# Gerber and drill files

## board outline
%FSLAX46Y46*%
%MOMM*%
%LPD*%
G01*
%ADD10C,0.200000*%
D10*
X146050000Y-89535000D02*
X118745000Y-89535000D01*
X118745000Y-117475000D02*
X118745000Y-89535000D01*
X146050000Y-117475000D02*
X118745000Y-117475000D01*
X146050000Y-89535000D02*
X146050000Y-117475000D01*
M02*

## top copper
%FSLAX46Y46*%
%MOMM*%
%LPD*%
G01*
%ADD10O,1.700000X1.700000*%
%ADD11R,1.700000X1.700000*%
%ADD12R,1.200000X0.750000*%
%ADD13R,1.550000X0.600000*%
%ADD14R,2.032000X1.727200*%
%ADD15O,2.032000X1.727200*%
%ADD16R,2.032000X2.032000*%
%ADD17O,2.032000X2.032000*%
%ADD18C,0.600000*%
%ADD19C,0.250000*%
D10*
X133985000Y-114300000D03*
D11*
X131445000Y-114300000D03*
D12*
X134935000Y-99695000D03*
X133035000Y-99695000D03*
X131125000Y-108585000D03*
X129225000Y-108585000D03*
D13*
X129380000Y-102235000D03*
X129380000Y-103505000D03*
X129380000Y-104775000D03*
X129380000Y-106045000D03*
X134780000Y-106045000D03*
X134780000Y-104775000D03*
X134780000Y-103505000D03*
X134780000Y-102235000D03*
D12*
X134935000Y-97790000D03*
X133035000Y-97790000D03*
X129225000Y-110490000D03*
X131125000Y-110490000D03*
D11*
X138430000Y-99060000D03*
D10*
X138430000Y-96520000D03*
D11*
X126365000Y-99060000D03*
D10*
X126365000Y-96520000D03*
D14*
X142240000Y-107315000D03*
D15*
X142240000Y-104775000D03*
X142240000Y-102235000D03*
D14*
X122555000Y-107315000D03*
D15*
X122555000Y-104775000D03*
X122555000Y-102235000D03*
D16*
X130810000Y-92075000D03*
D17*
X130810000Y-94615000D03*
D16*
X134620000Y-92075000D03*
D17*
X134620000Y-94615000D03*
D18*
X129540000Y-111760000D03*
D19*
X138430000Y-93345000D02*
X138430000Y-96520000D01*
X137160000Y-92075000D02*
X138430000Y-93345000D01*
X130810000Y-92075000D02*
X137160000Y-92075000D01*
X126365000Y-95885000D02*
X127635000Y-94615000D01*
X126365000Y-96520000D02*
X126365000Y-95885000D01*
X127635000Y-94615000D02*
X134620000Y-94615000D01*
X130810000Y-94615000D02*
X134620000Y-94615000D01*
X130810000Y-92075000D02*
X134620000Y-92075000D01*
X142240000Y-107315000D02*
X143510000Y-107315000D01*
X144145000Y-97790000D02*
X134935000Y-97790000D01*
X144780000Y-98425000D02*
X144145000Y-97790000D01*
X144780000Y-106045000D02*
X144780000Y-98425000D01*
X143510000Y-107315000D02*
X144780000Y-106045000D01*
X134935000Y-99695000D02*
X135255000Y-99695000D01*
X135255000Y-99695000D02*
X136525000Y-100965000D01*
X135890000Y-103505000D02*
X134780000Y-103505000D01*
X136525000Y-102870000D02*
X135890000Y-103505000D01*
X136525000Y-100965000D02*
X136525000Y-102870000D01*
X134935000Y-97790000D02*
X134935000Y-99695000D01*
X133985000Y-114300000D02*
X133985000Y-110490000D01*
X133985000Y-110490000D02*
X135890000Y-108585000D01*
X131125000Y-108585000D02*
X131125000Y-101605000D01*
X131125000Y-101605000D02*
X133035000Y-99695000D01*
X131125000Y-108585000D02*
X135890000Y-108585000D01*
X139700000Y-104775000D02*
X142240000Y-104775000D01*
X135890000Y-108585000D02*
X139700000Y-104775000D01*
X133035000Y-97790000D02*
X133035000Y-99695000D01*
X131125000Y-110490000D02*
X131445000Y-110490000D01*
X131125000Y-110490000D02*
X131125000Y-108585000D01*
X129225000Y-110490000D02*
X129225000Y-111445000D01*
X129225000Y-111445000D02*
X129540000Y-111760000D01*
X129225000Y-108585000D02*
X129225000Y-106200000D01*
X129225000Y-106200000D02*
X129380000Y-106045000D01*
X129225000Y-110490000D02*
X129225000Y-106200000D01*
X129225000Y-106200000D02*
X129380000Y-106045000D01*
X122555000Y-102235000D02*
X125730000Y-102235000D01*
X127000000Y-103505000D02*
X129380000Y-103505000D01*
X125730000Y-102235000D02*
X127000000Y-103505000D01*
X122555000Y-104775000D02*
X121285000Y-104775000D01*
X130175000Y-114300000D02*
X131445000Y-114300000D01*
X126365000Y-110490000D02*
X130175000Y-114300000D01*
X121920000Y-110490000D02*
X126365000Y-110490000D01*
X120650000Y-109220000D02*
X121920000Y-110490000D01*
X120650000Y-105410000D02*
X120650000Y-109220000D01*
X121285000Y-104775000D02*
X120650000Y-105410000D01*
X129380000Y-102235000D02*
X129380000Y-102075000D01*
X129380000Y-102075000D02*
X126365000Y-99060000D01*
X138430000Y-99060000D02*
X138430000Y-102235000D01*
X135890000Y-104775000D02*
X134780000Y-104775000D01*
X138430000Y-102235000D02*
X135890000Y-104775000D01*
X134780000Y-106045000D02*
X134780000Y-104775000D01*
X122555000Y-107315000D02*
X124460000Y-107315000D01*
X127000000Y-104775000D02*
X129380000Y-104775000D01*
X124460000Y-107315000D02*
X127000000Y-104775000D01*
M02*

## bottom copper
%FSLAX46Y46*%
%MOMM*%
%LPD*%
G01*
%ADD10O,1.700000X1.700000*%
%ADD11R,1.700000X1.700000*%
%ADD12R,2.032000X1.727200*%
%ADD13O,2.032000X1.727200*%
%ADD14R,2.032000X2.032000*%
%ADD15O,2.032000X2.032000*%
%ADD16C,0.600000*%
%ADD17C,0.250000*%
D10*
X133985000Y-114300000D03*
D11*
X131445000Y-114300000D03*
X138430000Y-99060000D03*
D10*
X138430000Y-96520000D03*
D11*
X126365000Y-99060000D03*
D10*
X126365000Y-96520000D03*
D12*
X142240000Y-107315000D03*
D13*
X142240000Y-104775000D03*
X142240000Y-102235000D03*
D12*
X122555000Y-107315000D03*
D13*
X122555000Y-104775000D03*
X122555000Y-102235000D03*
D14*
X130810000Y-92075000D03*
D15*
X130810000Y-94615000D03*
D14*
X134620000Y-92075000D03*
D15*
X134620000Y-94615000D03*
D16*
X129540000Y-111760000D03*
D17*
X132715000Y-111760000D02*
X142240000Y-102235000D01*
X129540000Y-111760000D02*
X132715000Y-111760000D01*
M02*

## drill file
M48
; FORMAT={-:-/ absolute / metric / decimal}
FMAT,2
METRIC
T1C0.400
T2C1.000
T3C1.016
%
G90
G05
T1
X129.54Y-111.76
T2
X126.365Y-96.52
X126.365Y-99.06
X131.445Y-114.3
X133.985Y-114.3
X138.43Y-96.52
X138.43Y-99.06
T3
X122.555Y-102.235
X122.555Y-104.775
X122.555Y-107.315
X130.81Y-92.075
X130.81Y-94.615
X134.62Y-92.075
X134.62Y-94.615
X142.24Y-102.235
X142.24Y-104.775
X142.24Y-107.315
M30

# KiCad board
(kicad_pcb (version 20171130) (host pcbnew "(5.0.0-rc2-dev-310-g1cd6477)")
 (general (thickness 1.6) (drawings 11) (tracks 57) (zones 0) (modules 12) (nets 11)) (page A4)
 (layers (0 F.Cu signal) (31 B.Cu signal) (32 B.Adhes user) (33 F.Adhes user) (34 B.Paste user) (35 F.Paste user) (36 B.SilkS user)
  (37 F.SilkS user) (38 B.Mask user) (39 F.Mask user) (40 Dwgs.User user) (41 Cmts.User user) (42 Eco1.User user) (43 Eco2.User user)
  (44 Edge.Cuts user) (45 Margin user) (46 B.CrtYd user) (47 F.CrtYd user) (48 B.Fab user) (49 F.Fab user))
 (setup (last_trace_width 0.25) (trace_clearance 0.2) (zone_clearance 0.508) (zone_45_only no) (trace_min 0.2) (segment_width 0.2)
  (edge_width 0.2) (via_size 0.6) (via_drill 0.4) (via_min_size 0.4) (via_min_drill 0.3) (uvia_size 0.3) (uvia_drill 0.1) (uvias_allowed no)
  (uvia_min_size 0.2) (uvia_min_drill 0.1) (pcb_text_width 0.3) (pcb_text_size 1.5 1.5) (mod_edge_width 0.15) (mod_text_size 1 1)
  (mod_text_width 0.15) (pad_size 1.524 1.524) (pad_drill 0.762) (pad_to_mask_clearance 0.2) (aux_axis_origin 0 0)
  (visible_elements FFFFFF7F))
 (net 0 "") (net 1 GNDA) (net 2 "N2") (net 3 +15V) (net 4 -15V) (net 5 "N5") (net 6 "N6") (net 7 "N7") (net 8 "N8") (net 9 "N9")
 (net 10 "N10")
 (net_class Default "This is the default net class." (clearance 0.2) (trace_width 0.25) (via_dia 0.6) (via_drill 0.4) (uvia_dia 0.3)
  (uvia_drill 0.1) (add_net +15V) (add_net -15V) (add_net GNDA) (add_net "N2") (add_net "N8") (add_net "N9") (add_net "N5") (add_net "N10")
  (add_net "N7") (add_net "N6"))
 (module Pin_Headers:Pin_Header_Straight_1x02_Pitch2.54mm (layer F.Cu) (at 131.445 114.3 90)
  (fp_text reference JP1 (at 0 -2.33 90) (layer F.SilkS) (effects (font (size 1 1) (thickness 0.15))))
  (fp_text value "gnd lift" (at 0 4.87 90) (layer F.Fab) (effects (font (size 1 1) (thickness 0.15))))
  (pad 2 thru_hole oval (at 0 2.54 90) (size 1.7 1.7) (drill 1) (layers *.Cu *.Mask) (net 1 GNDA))
  (pad 1 thru_hole rect (at 0 0 90) (size 1.7 1.7) (drill 1) (layers *.Cu *.Mask) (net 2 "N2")))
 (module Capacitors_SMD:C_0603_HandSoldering (layer F.Cu) (at 133.985 99.695 180)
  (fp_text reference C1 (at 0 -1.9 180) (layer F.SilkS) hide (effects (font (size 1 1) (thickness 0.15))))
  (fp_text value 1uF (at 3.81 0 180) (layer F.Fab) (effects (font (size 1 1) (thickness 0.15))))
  (pad 1 smd rect (at -0.95 0 180) (size 1.2 0.75) (layers F.Cu F.Paste F.Mask) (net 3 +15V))
  (pad 2 smd rect (at 0.95 0 180) (size 1.2 0.75) (layers F.Cu F.Paste F.Mask) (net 1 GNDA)))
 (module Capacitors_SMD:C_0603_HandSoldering (layer F.Cu) (at 130.175 108.585 180)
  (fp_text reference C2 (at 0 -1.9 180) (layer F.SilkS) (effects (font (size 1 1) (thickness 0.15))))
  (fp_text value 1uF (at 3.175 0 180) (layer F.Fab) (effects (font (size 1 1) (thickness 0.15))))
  (pad 1 smd rect (at -0.95 0 180) (size 1.2 0.75) (layers F.Cu F.Paste F.Mask) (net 1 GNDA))
  (pad 2 smd rect (at 0.95 0 180) (size 1.2 0.75) (layers F.Cu F.Paste F.Mask) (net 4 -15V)))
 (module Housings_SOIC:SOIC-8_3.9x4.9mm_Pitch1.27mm (layer F.Cu) (at 132.08 104.14)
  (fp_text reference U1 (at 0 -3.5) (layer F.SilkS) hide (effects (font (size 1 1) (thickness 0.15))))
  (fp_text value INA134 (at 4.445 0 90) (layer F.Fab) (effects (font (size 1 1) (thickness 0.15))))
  (pad 1 smd rect (at -2.7 -1.905) (size 1.55 0.6) (layers F.Cu F.Paste F.Mask) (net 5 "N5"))
  (pad 2 smd rect (at -2.7 -0.635) (size 1.55 0.6) (layers F.Cu F.Paste F.Mask) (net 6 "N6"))
  (pad 3 smd rect (at -2.7 0.635) (size 1.55 0.6) (layers F.Cu F.Paste F.Mask) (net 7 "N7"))
  (pad 4 smd rect (at -2.7 1.905) (size 1.55 0.6) (layers F.Cu F.Paste F.Mask) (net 4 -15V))
  (pad 5 smd rect (at 2.7 1.905) (size 1.55 0.6) (layers F.Cu F.Paste F.Mask) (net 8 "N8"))
  (pad 6 smd rect (at 2.7 0.635) (size 1.55 0.6) (layers F.Cu F.Paste F.Mask) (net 8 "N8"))
  (pad 7 smd rect (at 2.7 -0.635) (size 1.55 0.6) (layers F.Cu F.Paste F.Mask) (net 3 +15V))
  (pad 8 smd rect (at 2.7 -1.905) (size 1.55 0.6) (layers F.Cu F.Paste F.Mask)))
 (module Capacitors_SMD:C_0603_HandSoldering (layer F.Cu) (at 133.985 97.79 180)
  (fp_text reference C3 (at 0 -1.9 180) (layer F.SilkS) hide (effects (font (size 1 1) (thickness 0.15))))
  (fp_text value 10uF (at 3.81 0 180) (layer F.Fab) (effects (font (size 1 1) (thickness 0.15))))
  (pad 1 smd rect (at -0.95 0 180) (size 1.2 0.75) (layers F.Cu F.Paste F.Mask) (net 3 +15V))
  (pad 2 smd rect (at 0.95 0 180) (size 1.2 0.75) (layers F.Cu F.Paste F.Mask) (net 1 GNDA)))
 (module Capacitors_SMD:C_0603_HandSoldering (layer F.Cu) (at 130.175 110.49)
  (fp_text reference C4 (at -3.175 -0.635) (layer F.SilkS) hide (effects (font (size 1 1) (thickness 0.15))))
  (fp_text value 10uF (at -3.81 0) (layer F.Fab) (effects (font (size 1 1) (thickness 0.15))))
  (pad 1 smd rect (at -0.95 0) (size 1.2 0.75) (layers F.Cu F.Paste F.Mask) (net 4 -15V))
  (pad 2 smd rect (at 0.95 0) (size 1.2 0.75) (layers F.Cu F.Paste F.Mask) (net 1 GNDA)))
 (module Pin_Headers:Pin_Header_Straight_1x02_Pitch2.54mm (layer F.Cu) (at 138.43 99.06 180)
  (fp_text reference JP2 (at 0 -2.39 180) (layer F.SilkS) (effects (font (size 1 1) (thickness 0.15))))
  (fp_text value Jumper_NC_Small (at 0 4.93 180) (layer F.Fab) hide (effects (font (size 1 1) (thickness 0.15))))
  (pad 1 thru_hole rect (at 0 0 180) (size 1.7 1.7) (drill 1) (layers *.Cu *.Mask) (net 8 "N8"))
  (pad 2 thru_hole oval (at 0 2.54 180) (size 1.7 1.7) (drill 1) (layers *.Cu *.Mask) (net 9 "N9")))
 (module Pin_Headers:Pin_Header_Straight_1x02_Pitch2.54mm (layer F.Cu) (at 126.365 99.06 180)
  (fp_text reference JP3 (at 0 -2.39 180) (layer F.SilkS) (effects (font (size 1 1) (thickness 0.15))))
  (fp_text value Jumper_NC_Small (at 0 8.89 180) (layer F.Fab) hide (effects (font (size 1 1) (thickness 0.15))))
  (pad 1 thru_hole rect (at 0 0 180) (size 1.7 1.7) (drill 1) (layers *.Cu *.Mask) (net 5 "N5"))
  (pad 2 thru_hole oval (at 0 2.54 180) (size 1.7 1.7) (drill 1) (layers *.Cu *.Mask) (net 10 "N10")))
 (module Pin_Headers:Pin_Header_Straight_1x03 (layer F.Cu) (at 142.24 107.315 180)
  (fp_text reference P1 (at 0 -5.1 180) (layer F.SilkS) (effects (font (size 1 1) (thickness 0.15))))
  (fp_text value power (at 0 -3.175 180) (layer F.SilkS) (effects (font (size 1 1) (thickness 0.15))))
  (pad 1 thru_hole rect (at 0 0 180) (size 2.032 1.7272) (drill 1.016) (layers *.Cu *.Mask F.SilkS) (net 3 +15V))
  (pad 2 thru_hole oval (at 0 2.54 180) (size 2.032 1.7272) (drill 1.016) (layers *.Cu *.Mask F.SilkS) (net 1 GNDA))
  (pad 3 thru_hole oval (at 0 5.08 180) (size 2.032 1.7272) (drill 1.016) (layers *.Cu *.Mask F.SilkS) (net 4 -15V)))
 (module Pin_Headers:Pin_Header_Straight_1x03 (layer F.Cu) (at 122.555 107.315 180)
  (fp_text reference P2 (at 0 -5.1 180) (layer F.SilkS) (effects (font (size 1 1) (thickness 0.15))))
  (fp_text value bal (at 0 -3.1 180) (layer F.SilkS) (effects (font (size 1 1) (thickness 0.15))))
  (pad 1 thru_hole rect (at 0 0 180) (size 2.032 1.7272) (drill 1.016) (layers *.Cu *.Mask F.SilkS) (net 7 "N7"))
  (pad 2 thru_hole oval (at 0 2.54 180) (size 2.032 1.7272) (drill 1.016) (layers *.Cu *.Mask F.SilkS) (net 2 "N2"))
  (pad 3 thru_hole oval (at 0 5.08 180) (size 2.032 1.7272) (drill 1.016) (layers *.Cu *.Mask F.SilkS) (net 6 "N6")))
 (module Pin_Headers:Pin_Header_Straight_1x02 (layer F.Cu) (at 130.81 92.075)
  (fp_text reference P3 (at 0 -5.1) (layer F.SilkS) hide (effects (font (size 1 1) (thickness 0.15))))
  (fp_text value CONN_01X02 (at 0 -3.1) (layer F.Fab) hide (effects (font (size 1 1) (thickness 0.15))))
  (pad 1 thru_hole rect (at 0 0) (size 2.032 2.032) (drill 1.016) (layers *.Cu *.Mask F.SilkS) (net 9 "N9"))
  (pad 2 thru_hole oval (at 0 2.54) (size 2.032 2.032) (drill 1.016) (layers *.Cu *.Mask F.SilkS) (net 10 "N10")))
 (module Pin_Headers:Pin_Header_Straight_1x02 (layer F.Cu) (at 134.62 92.075)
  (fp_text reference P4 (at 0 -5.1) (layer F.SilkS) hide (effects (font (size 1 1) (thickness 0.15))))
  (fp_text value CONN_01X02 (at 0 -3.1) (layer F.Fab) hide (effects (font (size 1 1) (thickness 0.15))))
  (pad 1 thru_hole rect (at 0 0) (size 2.032 2.032) (drill 1.016) (layers *.Cu *.Mask F.SilkS) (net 9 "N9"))
  (pad 2 thru_hole oval (at 0 2.54) (size 2.032 2.032) (drill 1.016) (layers *.Cu *.Mask F.SilkS) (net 10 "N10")))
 (gr_line (start 146.05 89.535) (end 118.745 89.535) (angle 90) (layer Edge.Cuts) (width 0.2))
 (gr_line (start 118.745 117.475) (end 118.745 89.535) (angle 90) (layer Edge.Cuts) (width 0.2))
 (gr_line (start 146.05 117.475) (end 118.745 117.475) (angle 90) (layer Edge.Cuts) (width 0.2))
 (gr_line (start 146.05 89.535) (end 146.05 117.475) (angle 90) (layer Edge.Cuts) (width 0.2))
 (segment (start 138.43 93.345) (end 138.43 96.52) (width 0.25) (layer F.Cu) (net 9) (status 1000000))
 (segment (start 137.16 92.075) (end 138.43 93.345) (width 0.25) (layer F.Cu) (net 9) (status 1000000))
 (segment (start 130.81 92.075) (end 137.16 92.075) (width 0.25) (layer F.Cu) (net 9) (status 1000000))
 (segment (start 126.365 95.885) (end 127.635 94.615) (width 0.25) (layer F.Cu) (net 10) (status 1000000))
 (segment (start 126.365 96.52) (end 126.365 95.885) (width 0.25) (layer F.Cu) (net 10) (status 1000000))
 (segment (start 127.635 94.615) (end 134.62 94.615) (width 0.25) (layer F.Cu) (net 10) (status 1000000))
 (segment (start 130.81 94.615) (end 134.62 94.615) (width 0.25) (layer F.Cu) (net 10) (status 1000000))
 (segment (start 130.81 92.075) (end 134.62 92.075) (width 0.25) (layer F.Cu) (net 9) (status 1000000))
 (segment (start 142.24 107.315) (end 143.51 107.315) (width 0.25) (layer F.Cu) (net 3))
 (segment (start 144.145 97.79) (end 134.935 97.79) (width 0.25) (layer F.Cu) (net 3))
 (segment (start 144.78 98.425) (end 144.145 97.79) (width 0.25) (layer F.Cu) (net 3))
 (segment (start 144.78 106.045) (end 144.78 98.425) (width 0.25) (layer F.Cu) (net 3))
 (segment (start 143.51 107.315) (end 144.78 106.045) (width 0.25) (layer F.Cu) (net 3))
 (segment (start 134.935 99.695) (end 135.255 99.695) (width 0.25) (layer F.Cu) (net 3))
 (segment (start 135.255 99.695) (end 136.525 100.965) (width 0.25) (layer F.Cu) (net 3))
 (segment (start 135.89 103.505) (end 134.78 103.505) (width 0.25) (layer F.Cu) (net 3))
 (segment (start 136.525 102.87) (end 135.89 103.505) (width 0.25) (layer F.Cu) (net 3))
 (segment (start 136.525 100.965) (end 136.525 102.87) (width 0.25) (layer F.Cu) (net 3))
 (segment (start 134.935 97.79) (end 134.935 99.695) (width 0.25) (layer F.Cu) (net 3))
 (segment (start 133.985 114.3) (end 133.985 110.49) (width 0.25) (layer F.Cu) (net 1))
 (segment (start 133.985 110.49) (end 135.89 108.585) (width 0.25) (layer F.Cu) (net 1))
 (segment (start 131.125 108.585) (end 131.125 101.605) (width 0.25) (layer F.Cu) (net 1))
 (segment (start 131.125 101.605) (end 133.035 99.695) (width 0.25) (layer F.Cu) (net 1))
 (segment (start 131.125 108.585) (end 135.89 108.585) (width 0.25) (layer F.Cu) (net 1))
 (segment (start 139.7 104.775) (end 142.24 104.775) (width 0.25) (layer F.Cu) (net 1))
 (segment (start 135.89 108.585) (end 139.7 104.775) (width 0.25) (layer F.Cu) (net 1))
 (segment (start 133.035 97.79) (end 133.035 99.695) (width 0.25) (layer F.Cu) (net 1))
 (segment (start 131.125 110.49) (end 131.445 110.49) (width 0.25) (layer F.Cu) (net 1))
 (segment (start 131.125 110.49) (end 131.125 108.585) (width 0.25) (layer F.Cu) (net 1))
 (segment (start 129.225 110.49) (end 129.225 111.445) (width 0.25) (layer F.Cu) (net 4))
 (segment (start 132.715 111.76) (end 142.24 102.235) (width 0.25) (layer B.Cu) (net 4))
 (segment (start 129.54 111.76) (end 132.715 111.76) (width 0.25) (layer B.Cu) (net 4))
 (via (at 129.54 111.76) (size 0.6) (drill 0.4) (layers F.Cu B.Cu) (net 4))
 (segment (start 129.225 111.445) (end 129.54 111.76) (width 0.25) (layer F.Cu) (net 4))
 (segment (start 129.225 108.585) (end 129.225 106.2) (width 0.25) (layer F.Cu) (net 4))
 (segment (start 129.225 106.2) (end 129.38 106.045) (width 0.25) (layer F.Cu) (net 4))
 (segment (start 129.225 110.49) (end 129.225 106.2) (width 0.25) (layer F.Cu) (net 4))
 (segment (start 129.225 106.2) (end 129.38 106.045) (width 0.25) (layer F.Cu) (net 4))
 (segment (start 122.555 102.235) (end 125.73 102.235) (width 0.25) (layer F.Cu) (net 6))
 (segment (start 127 103.505) (end 129.38 103.505) (width 0.25) (layer F.Cu) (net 6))
 (segment (start 125.73 102.235) (end 127 103.505) (width 0.25) (layer F.Cu) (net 6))
 (segment (start 122.555 104.775) (end 121.285 104.775) (width 0.25) (layer F.Cu) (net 2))
 (segment (start 130.175 114.3) (end 131.445 114.3) (width 0.25) (layer F.Cu) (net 2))
 (segment (start 126.365 110.49) (end 130.175 114.3) (width 0.25) (layer F.Cu) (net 2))
 (segment (start 121.92 110.49) (end 126.365 110.49) (width 0.25) (layer F.Cu) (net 2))
 (segment (start 120.65 109.22) (end 121.92 110.49) (width 0.25) (layer F.Cu) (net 2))
 (segment (start 120.65 105.41) (end 120.65 109.22) (width 0.25) (layer F.Cu) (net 2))
 (segment (start 121.285 104.775) (end 120.65 105.41) (width 0.25) (layer F.Cu) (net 2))
 (segment (start 129.38 102.235) (end 129.38 102.075) (width 0.25) (layer F.Cu) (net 5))
 (segment (start 129.38 102.075) (end 126.365 99.06) (width 0.25) (layer F.Cu) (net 5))
 (segment (start 138.43 99.06) (end 138.43 102.235) (width 0.25) (layer F.Cu) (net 8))
 (segment (start 135.89 104.775) (end 134.78 104.775) (width 0.25) (layer F.Cu) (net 8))
 (segment (start 138.43 102.235) (end 135.89 104.775) (width 0.25) (layer F.Cu) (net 8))
 (segment (start 134.78 106.045) (end 134.78 104.775) (width 0.25) (layer F.Cu) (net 8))
 (segment (start 122.555 107.315) (end 124.46 107.315) (width 0.25) (layer F.Cu) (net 7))
 (segment (start 127 104.775) (end 129.38 104.775) (width 0.25) (layer F.Cu) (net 7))
 (segment (start 124.46 107.315) (end 127 104.775) (width 0.25) (layer F.Cu) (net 7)))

